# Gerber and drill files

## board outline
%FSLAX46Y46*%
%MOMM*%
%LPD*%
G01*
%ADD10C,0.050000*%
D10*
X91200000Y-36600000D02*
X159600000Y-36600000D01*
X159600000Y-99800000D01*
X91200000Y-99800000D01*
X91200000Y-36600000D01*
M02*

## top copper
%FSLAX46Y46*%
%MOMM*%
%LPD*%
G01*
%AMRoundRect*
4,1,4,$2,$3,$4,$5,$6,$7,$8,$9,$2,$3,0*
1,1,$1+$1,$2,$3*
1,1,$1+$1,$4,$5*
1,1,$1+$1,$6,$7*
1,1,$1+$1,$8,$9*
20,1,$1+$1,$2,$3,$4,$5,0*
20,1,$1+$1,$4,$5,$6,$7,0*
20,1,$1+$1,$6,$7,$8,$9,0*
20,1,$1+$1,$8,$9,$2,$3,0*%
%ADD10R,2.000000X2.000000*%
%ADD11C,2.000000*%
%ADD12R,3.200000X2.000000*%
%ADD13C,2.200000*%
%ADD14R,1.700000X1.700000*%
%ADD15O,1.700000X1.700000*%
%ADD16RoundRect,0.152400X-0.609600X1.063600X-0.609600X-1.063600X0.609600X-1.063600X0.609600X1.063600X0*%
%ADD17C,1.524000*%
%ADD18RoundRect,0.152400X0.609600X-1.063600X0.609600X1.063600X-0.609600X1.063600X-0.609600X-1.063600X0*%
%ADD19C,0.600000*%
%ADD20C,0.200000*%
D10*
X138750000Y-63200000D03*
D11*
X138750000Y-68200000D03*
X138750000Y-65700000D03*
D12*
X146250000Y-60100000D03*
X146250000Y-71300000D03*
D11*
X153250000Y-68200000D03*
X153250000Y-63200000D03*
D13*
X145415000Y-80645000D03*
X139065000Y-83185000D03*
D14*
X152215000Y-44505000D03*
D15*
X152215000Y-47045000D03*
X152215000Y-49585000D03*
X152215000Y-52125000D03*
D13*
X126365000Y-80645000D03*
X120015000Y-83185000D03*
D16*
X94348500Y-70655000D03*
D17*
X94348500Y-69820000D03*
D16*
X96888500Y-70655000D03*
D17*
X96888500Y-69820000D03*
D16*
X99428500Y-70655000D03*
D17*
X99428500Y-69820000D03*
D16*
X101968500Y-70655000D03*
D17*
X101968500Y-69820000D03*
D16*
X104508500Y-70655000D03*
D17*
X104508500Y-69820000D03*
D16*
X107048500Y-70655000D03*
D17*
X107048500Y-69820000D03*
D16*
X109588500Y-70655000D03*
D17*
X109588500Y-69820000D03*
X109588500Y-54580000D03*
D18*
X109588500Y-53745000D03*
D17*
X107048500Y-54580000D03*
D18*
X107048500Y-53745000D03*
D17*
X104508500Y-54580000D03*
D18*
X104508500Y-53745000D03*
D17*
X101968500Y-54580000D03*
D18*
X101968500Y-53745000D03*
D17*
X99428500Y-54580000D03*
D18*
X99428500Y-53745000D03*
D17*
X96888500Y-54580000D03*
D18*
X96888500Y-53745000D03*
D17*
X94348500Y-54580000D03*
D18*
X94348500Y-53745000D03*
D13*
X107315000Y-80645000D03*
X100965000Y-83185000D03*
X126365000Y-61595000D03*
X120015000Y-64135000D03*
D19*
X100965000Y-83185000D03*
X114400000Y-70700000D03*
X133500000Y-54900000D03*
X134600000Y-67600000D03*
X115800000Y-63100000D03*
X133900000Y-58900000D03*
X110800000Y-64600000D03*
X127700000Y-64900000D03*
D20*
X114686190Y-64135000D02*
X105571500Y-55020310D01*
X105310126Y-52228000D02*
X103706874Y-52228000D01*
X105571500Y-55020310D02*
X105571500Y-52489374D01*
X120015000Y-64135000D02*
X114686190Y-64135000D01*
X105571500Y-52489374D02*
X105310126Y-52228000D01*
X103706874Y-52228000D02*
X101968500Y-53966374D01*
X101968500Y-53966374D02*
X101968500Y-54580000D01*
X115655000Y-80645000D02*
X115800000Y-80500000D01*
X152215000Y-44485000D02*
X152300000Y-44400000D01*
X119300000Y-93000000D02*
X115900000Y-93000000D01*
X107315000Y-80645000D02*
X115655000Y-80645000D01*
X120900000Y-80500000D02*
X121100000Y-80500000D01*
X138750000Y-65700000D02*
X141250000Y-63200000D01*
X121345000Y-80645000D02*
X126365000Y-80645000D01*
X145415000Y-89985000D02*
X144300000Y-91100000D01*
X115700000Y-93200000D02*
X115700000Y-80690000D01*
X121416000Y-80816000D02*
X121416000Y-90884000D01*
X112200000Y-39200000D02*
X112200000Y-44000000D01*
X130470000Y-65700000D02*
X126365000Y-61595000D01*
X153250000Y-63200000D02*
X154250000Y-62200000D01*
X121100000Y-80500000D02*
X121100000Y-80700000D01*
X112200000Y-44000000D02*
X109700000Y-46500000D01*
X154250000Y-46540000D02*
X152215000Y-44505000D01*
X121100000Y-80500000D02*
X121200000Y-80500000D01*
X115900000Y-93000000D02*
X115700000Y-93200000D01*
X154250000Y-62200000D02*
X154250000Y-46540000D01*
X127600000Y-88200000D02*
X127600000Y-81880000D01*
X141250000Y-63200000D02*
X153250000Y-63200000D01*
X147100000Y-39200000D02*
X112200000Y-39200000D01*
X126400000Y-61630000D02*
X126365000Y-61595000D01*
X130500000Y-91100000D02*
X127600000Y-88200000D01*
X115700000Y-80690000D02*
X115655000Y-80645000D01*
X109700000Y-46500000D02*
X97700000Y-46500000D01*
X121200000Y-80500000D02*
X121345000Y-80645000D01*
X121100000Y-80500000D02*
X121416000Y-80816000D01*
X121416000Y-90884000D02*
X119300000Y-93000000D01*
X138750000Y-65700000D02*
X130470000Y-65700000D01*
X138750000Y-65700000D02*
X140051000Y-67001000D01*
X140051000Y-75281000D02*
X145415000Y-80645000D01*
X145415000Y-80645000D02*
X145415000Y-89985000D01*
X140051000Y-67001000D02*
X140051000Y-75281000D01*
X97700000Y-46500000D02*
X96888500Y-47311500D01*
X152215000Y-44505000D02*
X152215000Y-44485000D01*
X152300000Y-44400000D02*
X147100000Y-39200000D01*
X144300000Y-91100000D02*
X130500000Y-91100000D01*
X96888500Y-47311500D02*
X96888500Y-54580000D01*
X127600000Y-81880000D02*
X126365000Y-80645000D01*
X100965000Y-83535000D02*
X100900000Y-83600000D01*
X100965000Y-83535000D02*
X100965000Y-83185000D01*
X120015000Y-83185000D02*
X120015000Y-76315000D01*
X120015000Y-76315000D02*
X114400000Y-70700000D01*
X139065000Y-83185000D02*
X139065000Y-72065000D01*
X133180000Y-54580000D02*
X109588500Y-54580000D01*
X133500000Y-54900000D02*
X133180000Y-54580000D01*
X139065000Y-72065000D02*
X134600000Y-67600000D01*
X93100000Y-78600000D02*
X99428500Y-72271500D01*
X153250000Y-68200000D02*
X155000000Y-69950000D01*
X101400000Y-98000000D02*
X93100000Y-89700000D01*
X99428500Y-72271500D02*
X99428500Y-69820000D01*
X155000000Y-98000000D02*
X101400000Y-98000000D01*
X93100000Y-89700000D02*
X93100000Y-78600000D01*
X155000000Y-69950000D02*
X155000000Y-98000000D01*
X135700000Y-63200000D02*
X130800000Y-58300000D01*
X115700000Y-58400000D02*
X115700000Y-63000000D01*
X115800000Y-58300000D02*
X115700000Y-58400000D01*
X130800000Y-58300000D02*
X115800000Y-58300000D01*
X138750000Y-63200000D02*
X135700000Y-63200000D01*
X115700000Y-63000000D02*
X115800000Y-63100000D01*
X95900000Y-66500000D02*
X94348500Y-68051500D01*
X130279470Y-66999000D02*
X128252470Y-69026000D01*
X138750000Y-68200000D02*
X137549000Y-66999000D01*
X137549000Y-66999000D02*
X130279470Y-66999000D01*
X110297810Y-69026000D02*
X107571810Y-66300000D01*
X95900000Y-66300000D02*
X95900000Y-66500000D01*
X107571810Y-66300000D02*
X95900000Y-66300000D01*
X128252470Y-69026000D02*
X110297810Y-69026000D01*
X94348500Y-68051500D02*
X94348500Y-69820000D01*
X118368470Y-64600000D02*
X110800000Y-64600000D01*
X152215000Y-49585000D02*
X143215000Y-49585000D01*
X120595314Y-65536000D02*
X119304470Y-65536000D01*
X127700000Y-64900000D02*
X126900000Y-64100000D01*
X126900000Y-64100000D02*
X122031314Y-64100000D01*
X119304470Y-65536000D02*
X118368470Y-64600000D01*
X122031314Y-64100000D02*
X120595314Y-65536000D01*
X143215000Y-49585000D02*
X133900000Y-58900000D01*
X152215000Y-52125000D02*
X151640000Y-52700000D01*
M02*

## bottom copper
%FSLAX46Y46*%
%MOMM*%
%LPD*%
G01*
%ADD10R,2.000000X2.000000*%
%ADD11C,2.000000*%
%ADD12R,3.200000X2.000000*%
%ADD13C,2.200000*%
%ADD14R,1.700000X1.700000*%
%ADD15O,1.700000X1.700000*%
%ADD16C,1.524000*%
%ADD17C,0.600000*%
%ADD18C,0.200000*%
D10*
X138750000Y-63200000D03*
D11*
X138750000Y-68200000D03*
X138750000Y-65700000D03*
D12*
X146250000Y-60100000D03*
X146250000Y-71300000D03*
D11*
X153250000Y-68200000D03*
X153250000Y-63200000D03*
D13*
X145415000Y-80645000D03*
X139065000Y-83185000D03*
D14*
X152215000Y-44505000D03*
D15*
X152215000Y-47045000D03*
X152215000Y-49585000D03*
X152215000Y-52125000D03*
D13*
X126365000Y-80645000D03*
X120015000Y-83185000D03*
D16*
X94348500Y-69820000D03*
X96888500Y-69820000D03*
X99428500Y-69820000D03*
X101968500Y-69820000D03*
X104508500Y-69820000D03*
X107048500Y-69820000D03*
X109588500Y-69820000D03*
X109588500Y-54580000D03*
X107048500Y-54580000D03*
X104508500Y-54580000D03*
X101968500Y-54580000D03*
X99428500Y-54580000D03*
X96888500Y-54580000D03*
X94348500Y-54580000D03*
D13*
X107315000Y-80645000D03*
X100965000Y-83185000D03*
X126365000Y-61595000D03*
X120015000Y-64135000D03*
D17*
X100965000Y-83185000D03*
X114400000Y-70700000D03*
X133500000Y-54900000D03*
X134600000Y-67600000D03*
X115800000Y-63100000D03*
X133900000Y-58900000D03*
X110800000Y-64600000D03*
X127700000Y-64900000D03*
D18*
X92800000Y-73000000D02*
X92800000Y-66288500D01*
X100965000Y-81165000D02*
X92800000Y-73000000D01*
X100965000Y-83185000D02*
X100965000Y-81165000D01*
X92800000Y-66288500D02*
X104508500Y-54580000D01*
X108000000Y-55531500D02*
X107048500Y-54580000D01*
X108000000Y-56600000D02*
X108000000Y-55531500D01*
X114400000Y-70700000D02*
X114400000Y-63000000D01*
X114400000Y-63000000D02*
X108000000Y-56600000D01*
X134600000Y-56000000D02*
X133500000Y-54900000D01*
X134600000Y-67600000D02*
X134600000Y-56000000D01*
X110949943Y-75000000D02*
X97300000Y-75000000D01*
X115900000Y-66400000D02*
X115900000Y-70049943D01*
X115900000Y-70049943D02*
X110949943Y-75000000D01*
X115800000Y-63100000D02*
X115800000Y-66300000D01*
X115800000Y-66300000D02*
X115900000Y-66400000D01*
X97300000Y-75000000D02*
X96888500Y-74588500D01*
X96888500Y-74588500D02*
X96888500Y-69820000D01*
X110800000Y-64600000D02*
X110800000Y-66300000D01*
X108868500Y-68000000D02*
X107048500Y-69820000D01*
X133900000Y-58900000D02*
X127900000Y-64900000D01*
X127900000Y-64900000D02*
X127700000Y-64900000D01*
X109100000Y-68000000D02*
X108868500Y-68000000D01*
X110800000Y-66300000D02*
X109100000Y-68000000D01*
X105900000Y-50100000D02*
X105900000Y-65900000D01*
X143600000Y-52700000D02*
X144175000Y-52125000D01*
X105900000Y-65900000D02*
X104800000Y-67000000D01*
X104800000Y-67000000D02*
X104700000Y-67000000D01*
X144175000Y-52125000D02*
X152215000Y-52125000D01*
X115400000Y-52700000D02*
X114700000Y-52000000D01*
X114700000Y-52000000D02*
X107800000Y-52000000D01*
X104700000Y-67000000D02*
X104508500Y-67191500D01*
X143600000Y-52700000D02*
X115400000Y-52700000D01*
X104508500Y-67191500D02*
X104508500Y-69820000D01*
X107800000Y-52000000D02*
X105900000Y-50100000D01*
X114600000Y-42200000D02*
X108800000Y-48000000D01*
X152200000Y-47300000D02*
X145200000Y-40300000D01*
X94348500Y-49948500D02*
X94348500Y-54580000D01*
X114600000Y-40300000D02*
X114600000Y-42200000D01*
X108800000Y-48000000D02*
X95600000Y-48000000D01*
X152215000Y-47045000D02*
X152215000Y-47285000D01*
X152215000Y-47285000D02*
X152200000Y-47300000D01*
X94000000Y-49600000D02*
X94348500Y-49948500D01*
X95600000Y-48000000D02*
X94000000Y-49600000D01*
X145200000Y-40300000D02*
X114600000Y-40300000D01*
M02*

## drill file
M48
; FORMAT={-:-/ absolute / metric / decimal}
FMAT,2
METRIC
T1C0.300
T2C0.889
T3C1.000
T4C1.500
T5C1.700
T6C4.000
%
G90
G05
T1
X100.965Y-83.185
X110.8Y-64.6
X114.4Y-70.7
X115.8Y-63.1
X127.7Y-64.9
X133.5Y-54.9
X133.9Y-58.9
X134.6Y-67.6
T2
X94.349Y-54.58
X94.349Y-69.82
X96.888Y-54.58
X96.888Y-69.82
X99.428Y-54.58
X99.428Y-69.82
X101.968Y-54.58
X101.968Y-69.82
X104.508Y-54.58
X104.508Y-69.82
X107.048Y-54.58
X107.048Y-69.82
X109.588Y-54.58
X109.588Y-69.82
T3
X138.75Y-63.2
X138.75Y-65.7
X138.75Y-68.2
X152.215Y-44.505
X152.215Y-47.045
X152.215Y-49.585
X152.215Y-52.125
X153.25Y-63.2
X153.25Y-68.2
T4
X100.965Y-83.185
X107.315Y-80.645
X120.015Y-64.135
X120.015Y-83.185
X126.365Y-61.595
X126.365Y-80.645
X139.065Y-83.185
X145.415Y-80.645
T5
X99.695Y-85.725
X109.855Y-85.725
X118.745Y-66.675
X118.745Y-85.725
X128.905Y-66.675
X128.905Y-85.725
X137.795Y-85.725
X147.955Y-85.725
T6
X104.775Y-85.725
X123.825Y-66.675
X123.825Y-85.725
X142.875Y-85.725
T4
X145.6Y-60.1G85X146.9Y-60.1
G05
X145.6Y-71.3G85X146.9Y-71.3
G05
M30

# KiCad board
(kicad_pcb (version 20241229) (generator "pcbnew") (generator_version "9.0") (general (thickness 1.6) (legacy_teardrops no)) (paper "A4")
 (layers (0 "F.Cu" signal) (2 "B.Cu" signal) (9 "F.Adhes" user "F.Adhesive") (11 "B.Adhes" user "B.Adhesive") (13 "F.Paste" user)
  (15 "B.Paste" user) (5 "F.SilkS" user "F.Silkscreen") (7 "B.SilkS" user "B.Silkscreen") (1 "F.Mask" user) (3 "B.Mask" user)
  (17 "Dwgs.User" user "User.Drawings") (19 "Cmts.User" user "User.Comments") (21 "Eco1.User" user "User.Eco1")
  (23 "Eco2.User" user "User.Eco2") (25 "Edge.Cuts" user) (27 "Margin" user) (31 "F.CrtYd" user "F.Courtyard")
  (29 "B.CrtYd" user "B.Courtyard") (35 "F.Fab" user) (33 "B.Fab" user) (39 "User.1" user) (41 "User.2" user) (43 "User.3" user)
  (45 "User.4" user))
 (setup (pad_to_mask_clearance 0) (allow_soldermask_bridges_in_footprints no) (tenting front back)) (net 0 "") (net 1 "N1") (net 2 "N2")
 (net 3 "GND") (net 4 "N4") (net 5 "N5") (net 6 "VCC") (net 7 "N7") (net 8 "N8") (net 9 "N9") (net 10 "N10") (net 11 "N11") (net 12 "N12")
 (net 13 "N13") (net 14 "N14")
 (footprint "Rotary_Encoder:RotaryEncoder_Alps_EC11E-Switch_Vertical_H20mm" (layer "F.Cu") (at 138.75 63.2)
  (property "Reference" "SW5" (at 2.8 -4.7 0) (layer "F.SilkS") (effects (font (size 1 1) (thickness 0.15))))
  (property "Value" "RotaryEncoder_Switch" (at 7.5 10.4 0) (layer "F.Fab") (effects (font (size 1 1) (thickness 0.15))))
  (pad "A" thru_hole rect (at 0 0) (size 2 2) (drill 1) (layers "*.Cu" "*.Mask") (remove_unused_layers no) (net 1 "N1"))
  (pad "B" thru_hole circle (at 0 5) (size 2 2) (drill 1) (layers "*.Cu" "*.Mask") (remove_unused_layers no) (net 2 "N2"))
  (pad "C" thru_hole circle (at 0 2.5) (size 2 2) (drill 1) (layers "*.Cu" "*.Mask") (remove_unused_layers no) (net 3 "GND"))
  (pad "MP" thru_hole rect (at 7.5 -3.1) (size 3.2 2) (drill oval 2.8 1.5) (layers "*.Cu" "*.Mask") (remove_unused_layers no))
  (pad "MP" thru_hole rect (at 7.5 8.1) (size 3.2 2) (drill oval 2.8 1.5) (layers "*.Cu" "*.Mask") (remove_unused_layers no))
  (pad "S1" thru_hole circle (at 14.5 5) (size 2 2) (drill 1) (layers "*.Cu" "*.Mask") (remove_unused_layers no) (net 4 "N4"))
  (pad "S2" thru_hole circle (at 14.5 0) (size 2 2) (drill 1) (layers "*.Cu" "*.Mask") (remove_unused_layers no) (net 3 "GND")))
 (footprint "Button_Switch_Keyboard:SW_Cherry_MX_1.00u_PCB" (layer "F.Cu") (at 145.415 80.645)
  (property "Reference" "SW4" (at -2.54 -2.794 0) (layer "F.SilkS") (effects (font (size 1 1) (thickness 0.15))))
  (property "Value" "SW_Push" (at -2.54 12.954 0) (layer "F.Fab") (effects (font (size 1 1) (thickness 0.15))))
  (pad "" np_thru_hole circle (at -7.62 5.08) (size 1.7 1.7) (drill 1.7) (layers "*.Cu" "*.Mask"))
  (pad "" np_thru_hole circle (at -2.54 5.08) (size 4 4) (drill 4) (layers "*.Cu" "*.Mask"))
  (pad "" np_thru_hole circle (at 2.54 5.08) (size 1.7 1.7) (drill 1.7) (layers "*.Cu" "*.Mask"))
  (pad "1" thru_hole circle (at 0 0) (size 2.2 2.2) (drill 1.5) (layers "*.Cu" "*.Mask") (remove_unused_layers no) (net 3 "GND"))
  (pad "2" thru_hole circle (at -6.35 2.54) (size 2.2 2.2) (drill 1.5) (layers "*.Cu" "*.Mask") (remove_unused_layers no) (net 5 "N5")))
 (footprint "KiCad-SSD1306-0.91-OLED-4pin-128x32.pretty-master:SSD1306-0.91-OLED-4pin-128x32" (layer "F.Cu") (at 115.715 42.315)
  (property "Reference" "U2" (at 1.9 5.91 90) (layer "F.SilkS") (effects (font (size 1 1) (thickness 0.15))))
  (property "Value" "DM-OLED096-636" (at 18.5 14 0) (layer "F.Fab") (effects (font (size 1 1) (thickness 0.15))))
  (pad "1" thru_hole rect (at 36.5 2.19) (size 1.7 1.7) (drill 1) (layers "*.Cu" "*.Mask") (remove_unused_layers no) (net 3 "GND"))
  (pad "2" thru_hole oval (at 36.5 4.73) (size 1.7 1.7) (drill 1) (layers "*.Cu" "*.Mask") (remove_unused_layers no) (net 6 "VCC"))
  (pad "3" thru_hole oval (at 36.5 7.27) (size 1.7 1.7) (drill 1) (layers "*.Cu" "*.Mask") (remove_unused_layers no) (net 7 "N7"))
  (pad "4" thru_hole oval (at 36.5 9.81) (size 1.7 1.7) (drill 1) (layers "*.Cu" "*.Mask") (remove_unused_layers no) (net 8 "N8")))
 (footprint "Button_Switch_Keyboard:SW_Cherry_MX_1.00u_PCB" (layer "F.Cu") (at 126.365 80.645)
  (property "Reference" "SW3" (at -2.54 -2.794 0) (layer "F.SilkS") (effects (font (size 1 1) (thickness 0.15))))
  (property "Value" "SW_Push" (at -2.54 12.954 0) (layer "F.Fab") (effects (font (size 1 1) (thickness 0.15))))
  (pad "" np_thru_hole circle (at -7.62 5.08) (size 1.7 1.7) (drill 1.7) (layers "*.Cu" "*.Mask"))
  (pad "" np_thru_hole circle (at -2.54 5.08) (size 4 4) (drill 4) (layers "*.Cu" "*.Mask"))
  (pad "" np_thru_hole circle (at 2.54 5.08) (size 1.7 1.7) (drill 1.7) (layers "*.Cu" "*.Mask"))
  (pad "1" thru_hole circle (at 0 0) (size 2.2 2.2) (drill 1.5) (layers "*.Cu" "*.Mask") (remove_unused_layers no) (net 3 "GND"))
  (pad "2" thru_hole circle (at -6.35 2.54) (size 2.2 2.2) (drill 1.5) (layers "*.Cu" "*.Mask") (remove_unused_layers no) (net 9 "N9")))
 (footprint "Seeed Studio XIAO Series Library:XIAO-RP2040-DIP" (layer "F.Cu") (at 101.9685 62.2 90)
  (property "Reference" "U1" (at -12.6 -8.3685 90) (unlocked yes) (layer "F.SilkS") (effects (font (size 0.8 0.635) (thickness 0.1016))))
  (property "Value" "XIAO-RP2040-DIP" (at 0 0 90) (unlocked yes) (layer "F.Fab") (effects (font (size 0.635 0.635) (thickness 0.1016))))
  (pad "1" smd roundrect (at -8.455 -7.62 270) (size 2.432 1.524) (layers "F.Cu" "F.Mask") (roundrect_rratio 0.1) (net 2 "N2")
   (thermal_bridge_angle 45))
  (pad "1" thru_hole circle (at -7.62 -7.62 270) (size 1.524 1.524) (drill 0.889) (layers "*.Cu" "*.Mask") (remove_unused_layers no)
   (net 2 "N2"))
  (pad "2" smd roundrect (at -8.455 -5.08 270) (size 2.432 1.524) (layers "F.Cu" "F.Mask") (roundrect_rratio 0.1) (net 1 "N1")
   (thermal_bridge_angle 45))
  (pad "2" thru_hole circle (at -7.62 -5.08 270) (size 1.524 1.524) (drill 0.889) (layers "*.Cu" "*.Mask") (remove_unused_layers no)
   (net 1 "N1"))
  (pad "3" smd roundrect (at -8.455 -2.54 270) (size 2.432 1.524) (layers "F.Cu" "F.Mask") (roundrect_rratio 0.1) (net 4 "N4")
   (thermal_bridge_angle 45))
  (pad "3" thru_hole circle (at -7.62 -2.54 270) (size 1.524 1.524) (drill 0.889) (layers "*.Cu" "*.Mask") (remove_unused_layers no)
   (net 4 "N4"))
  (pad "4" smd roundrect (at -8.455 0 270) (size 2.432 1.524) (layers "F.Cu" "F.Mask") (roundrect_rratio 0.1) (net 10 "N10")
   (thermal_bridge_angle 45))
  (pad "4" thru_hole circle (at -7.62 0 270) (size 1.524 1.524) (drill 0.889) (layers "*.Cu" "*.Mask") (remove_unused_layers no)
   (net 10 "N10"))
  (pad "5" smd roundrect (at -8.455 2.54 270) (size 2.432 1.524) (layers "F.Cu" "F.Mask") (roundrect_rratio 0.1) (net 8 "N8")
   (thermal_bridge_angle 45))
  (pad "5" thru_hole circle (at -7.62 2.54 270) (size 1.524 1.524) (drill 0.889) (layers "*.Cu" "*.Mask") (remove_unused_layers no)
   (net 8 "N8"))
  (pad "6" smd roundrect (at -8.455 5.08 270) (size 2.432 1.524) (layers "F.Cu" "F.Mask") (roundrect_rratio 0.1) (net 7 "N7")
   (thermal_bridge_angle 45))
  (pad "6" thru_hole circle (at -7.62 5.08 270) (size 1.524 1.524) (drill 0.889) (layers "*.Cu" "*.Mask") (remove_unused_layers no)
   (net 7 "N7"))
  (pad "7" smd roundrect (at -8.455 7.62 270) (size 2.432 1.524) (layers "F.Cu" "F.Mask") (roundrect_rratio 0.1) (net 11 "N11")
   (thermal_bridge_angle 45))
  (pad "7" thru_hole circle (at -7.62 7.62 270) (size 1.524 1.524) (drill 0.889) (layers "*.Cu" "*.Mask") (remove_unused_layers no)
   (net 11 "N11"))
  (pad "8" thru_hole circle (at 7.62 7.62 90) (size 1.524 1.524) (drill 0.889) (layers "*.Cu" "*.Mask") (remove_unused_layers no)
   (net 5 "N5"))
  (pad "8" smd roundrect (at 8.455 7.62 90) (size 2.432 1.524) (layers "F.Cu" "F.Mask") (roundrect_rratio 0.1) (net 5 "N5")
   (thermal_bridge_angle 45))
  (pad "9" thru_hole circle (at 7.62 5.08 90) (size 1.524 1.524) (drill 0.889) (layers "*.Cu" "*.Mask") (remove_unused_layers no)
   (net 9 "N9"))
  (pad "9" smd roundrect (at 8.455 5.08 90) (size 2.432 1.524) (layers "F.Cu" "F.Mask") (roundrect_rratio 0.1) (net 9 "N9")
   (thermal_bridge_angle 45))
  (pad "10" thru_hole circle (at 7.62 2.54 90) (size 1.524 1.524) (drill 0.889) (layers "*.Cu" "*.Mask") (remove_unused_layers no)
   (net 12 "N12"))
  (pad "10" smd roundrect (at 8.455 2.54 90) (size 2.432 1.524) (layers "F.Cu" "F.Mask") (roundrect_rratio 0.1) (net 12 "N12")
   (thermal_bridge_angle 45))
  (pad "11" thru_hole circle (at 7.62 0 90) (size 1.524 1.524) (drill 0.889) (layers "*.Cu" "*.Mask") (remove_unused_layers no)
   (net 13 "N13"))
  (pad "11" smd roundrect (at 8.455 0 90) (size 2.432 1.524) (layers "F.Cu" "F.Mask") (roundrect_rratio 0.1) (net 13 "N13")
   (thermal_bridge_angle 45))
  (pad "12" thru_hole circle (at 7.62 -2.54 90) (size 1.524 1.524) (drill 0.889) (layers "*.Cu" "*.Mask") (remove_unused_layers no)
   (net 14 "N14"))
  (pad "12" smd roundrect (at 8.455 -2.54 90) (size 2.432 1.524) (layers "F.Cu" "F.Mask") (roundrect_rratio 0.1) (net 14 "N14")
   (thermal_bridge_angle 45))
  (pad "13" thru_hole circle (at 7.62 -5.08 90) (size 1.524 1.524) (drill 0.889) (layers "*.Cu" "*.Mask") (remove_unused_layers no)
   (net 3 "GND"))
  (pad "13" smd roundrect (at 8.455 -5.08 90) (size 2.432 1.524) (layers "F.Cu" "F.Mask") (roundrect_rratio 0.1) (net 3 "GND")
   (thermal_bridge_angle 45))
  (pad "14" thru_hole circle (at 7.62 -7.62 90) (size 1.524 1.524) (drill 0.889) (layers "*.Cu" "*.Mask") (remove_unused_layers no)
   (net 6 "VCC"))
  (pad "14" smd roundrect (at 8.455 -7.62 90) (size 2.432 1.524) (layers "F.Cu" "F.Mask") (roundrect_rratio 0.1) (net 6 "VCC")
   (thermal_bridge_angle 45)))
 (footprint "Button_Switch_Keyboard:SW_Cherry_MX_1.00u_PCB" (layer "F.Cu") (at 107.315 80.645)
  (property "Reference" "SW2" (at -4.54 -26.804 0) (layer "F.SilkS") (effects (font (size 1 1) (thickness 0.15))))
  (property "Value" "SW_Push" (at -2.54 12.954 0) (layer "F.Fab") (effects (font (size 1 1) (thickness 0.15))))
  (pad "" np_thru_hole circle (at -7.62 5.08) (size 1.7 1.7) (drill 1.7) (layers "*.Cu" "*.Mask"))
  (pad "" np_thru_hole circle (at -2.54 5.08) (size 4 4) (drill 4) (layers "*.Cu" "*.Mask"))
  (pad "" np_thru_hole circle (at 2.54 5.08) (size 1.7 1.7) (drill 1.7) (layers "*.Cu" "*.Mask"))
  (pad "1" thru_hole circle (at 0 0) (size 2.2 2.2) (drill 1.5) (layers "*.Cu" "*.Mask") (remove_unused_layers no) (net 3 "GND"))
  (pad "2" thru_hole circle (at -6.35 2.54) (size 2.2 2.2) (drill 1.5) (layers "*.Cu" "*.Mask") (remove_unused_layers no) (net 12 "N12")))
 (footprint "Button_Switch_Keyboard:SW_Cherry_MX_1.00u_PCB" (layer "F.Cu") (at 126.365 61.595)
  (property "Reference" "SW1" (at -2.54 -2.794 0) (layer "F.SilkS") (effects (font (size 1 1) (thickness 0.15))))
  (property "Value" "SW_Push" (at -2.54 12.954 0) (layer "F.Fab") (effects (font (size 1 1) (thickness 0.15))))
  (pad "" np_thru_hole circle (at -7.62 5.08) (size 1.7 1.7) (drill 1.7) (layers "*.Cu" "*.Mask"))
  (pad "" np_thru_hole circle (at -2.54 5.08) (size 4 4) (drill 4) (layers "*.Cu" "*.Mask"))
  (pad "" np_thru_hole circle (at 2.54 5.08) (size 1.7 1.7) (drill 1.7) (layers "*.Cu" "*.Mask"))
  (pad "1" thru_hole circle (at 0 0) (size 2.2 2.2) (drill 1.5) (layers "*.Cu" "*.Mask") (remove_unused_layers no) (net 3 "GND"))
  (pad "2" thru_hole circle (at -6.35 2.54) (size 2.2 2.2) (drill 1.5) (layers "*.Cu" "*.Mask") (remove_unused_layers no) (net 13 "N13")))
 (gr_rect (start 91.2 36.6) (end 159.6 99.8) (stroke (width 0.05) (type default)) (fill no) (layer "Edge.Cuts"))
 (segment (start 114.68619 64.135) (end 105.5715 55.02031) (width 0.2) (layer "F.Cu") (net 13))
 (segment (start 105.310126 52.228) (end 103.706874 52.228) (width 0.2) (layer "F.Cu") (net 13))
 (segment (start 105.5715 55.02031) (end 105.5715 52.489374) (width 0.2) (layer "F.Cu") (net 13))
 (segment (start 120.015 64.135) (end 114.68619 64.135) (width 0.2) (layer "F.Cu") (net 13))
 (segment (start 105.5715 52.489374) (end 105.310126 52.228) (width 0.2) (layer "F.Cu") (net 13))
 (segment (start 103.706874 52.228) (end 101.9685 53.966374) (width 0.2) (layer "F.Cu") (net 13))
 (segment (start 101.9685 53.966374) (end 101.9685 54.58) (width 0.2) (layer "F.Cu") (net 13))
 (segment (start 115.655 80.645) (end 115.8 80.5) (width 0.2) (layer "F.Cu") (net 3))
 (segment (start 152.215 44.485) (end 152.3 44.4) (width 0.2) (layer "F.Cu") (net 3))
 (segment (start 119.3 93) (end 115.9 93) (width 0.2) (layer "F.Cu") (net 3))
 (segment (start 107.315 80.645) (end 115.655 80.645) (width 0.2) (layer "F.Cu") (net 3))
 (segment (start 120.9 80.5) (end 121.1 80.5) (width 0.2) (layer "F.Cu") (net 3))
 (segment (start 138.75 65.7) (end 141.25 63.2) (width 0.2) (layer "F.Cu") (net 3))
 (segment (start 121.345 80.645) (end 126.365 80.645) (width 0.2) (layer "F.Cu") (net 3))
 (segment (start 145.415 89.985) (end 144.3 91.1) (width 0.2) (layer "F.Cu") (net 3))
 (segment (start 115.7 93.2) (end 115.7 80.69) (width 0.2) (layer "F.Cu") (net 3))
 (segment (start 121.416 80.816) (end 121.416 90.884) (width 0.2) (layer "F.Cu") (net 3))
 (segment (start 112.2 39.2) (end 112.2 44) (width 0.2) (layer "F.Cu") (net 3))
 (segment (start 130.47 65.7) (end 126.365 61.595) (width 0.2) (layer "F.Cu") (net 3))
 (segment (start 153.25 63.2) (end 154.25 62.2) (width 0.2) (layer "F.Cu") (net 3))
 (segment (start 121.1 80.5) (end 121.1 80.7) (width 0.2) (layer "F.Cu") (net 3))
 (segment (start 112.2 44) (end 109.7 46.5) (width 0.2) (layer "F.Cu") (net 3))
 (segment (start 154.25 46.54) (end 152.215 44.505) (width 0.2) (layer "F.Cu") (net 3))
 (segment (start 121.1 80.5) (end 121.2 80.5) (width 0.2) (layer "F.Cu") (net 3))
 (segment (start 115.9 93) (end 115.7 93.2) (width 0.2) (layer "F.Cu") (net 3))
 (segment (start 154.25 62.2) (end 154.25 46.54) (width 0.2) (layer "F.Cu") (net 3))
 (segment (start 127.6 88.2) (end 127.6 81.88) (width 0.2) (layer "F.Cu") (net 3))
 (segment (start 141.25 63.2) (end 153.25 63.2) (width 0.2) (layer "F.Cu") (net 3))
 (segment (start 147.1 39.2) (end 112.2 39.2) (width 0.2) (layer "F.Cu") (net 3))
 (segment (start 126.4 61.63) (end 126.365 61.595) (width 0.2) (layer "F.Cu") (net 3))
 (segment (start 130.5 91.1) (end 127.6 88.2) (width 0.2) (layer "F.Cu") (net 3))
 (segment (start 115.7 80.69) (end 115.655 80.645) (width 0.2) (layer "F.Cu") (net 3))
 (segment (start 109.7 46.5) (end 97.7 46.5) (width 0.2) (layer "F.Cu") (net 3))
 (segment (start 121.2 80.5) (end 121.345 80.645) (width 0.2) (layer "F.Cu") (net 3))
 (segment (start 121.1 80.5) (end 121.416 80.816) (width 0.2) (layer "F.Cu") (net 3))
 (segment (start 121.416 90.884) (end 119.3 93) (width 0.2) (layer "F.Cu") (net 3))
 (segment (start 138.75 65.7) (end 130.47 65.7) (width 0.2) (layer "F.Cu") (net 3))
 (segment (start 138.75 65.7) (end 140.051 67.001) (width 0.2) (layer "F.Cu") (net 3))
 (segment (start 140.051 75.281) (end 145.415 80.645) (width 0.2) (layer "F.Cu") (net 3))
 (segment (start 145.415 80.645) (end 145.415 89.985) (width 0.2) (layer "F.Cu") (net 3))
 (segment (start 140.051 67.001) (end 140.051 75.281) (width 0.2) (layer "F.Cu") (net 3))
 (segment (start 97.7 46.5) (end 96.8885 47.3115) (width 0.2) (layer "F.Cu") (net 3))
 (segment (start 152.215 44.505) (end 152.215 44.485) (width 0.2) (layer "F.Cu") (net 3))
 (segment (start 152.3 44.4) (end 147.1 39.2) (width 0.2) (layer "F.Cu") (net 3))
 (segment (start 144.3 91.1) (end 130.5 91.1) (width 0.2) (layer "F.Cu") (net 3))
 (segment (start 96.8885 47.3115) (end 96.8885 54.58) (width 0.2) (layer "F.Cu") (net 3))
 (segment (start 127.6 81.88) (end 126.365 80.645) (width 0.2) (layer "F.Cu") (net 3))
 (segment (start 100.965 83.535) (end 100.9 83.6) (width 0.2) (layer "F.Cu") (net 12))
 (segment (start 100.965 83.535) (end 100.965 83.185) (width 0.2) (layer "F.Cu") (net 12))
 (via (at 100.965 83.185) (size 0.6) (drill 0.3) (layers "F.Cu" "B.Cu") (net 12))
 (segment (start 92.8 73) (end 92.8 66.2885) (width 0.2) (layer "B.Cu") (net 12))
 (segment (start 100.965 81.165) (end 92.8 73) (width 0.2) (layer "B.Cu") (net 12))
 (segment (start 100.965 83.185) (end 100.965 81.165) (width 0.2) (layer "B.Cu") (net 12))
 (segment (start 92.8 66.2885) (end 104.5085 54.58) (width 0.2) (layer "B.Cu") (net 12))
 (segment (start 120.015 83.185) (end 120.015 76.315) (width 0.2) (layer "F.Cu") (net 9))
 (segment (start 120.015 76.315) (end 114.4 70.7) (width 0.2) (layer "F.Cu") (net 9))
 (via (at 114.4 70.7) (size 0.6) (drill 0.3) (layers "F.Cu" "B.Cu") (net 9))
 (segment (start 108 55.5315) (end 107.0485 54.58) (width 0.2) (layer "B.Cu") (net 9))
 (segment (start 108 56.6) (end 108 55.5315) (width 0.2) (layer "B.Cu") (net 9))
 (segment (start 114.4 70.7) (end 114.4 63) (width 0.2) (layer "B.Cu") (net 9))
 (segment (start 114.4 63) (end 108 56.6) (width 0.2) (layer "B.Cu") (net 9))
 (segment (start 139.065 83.185) (end 139.065 72.065) (width 0.2) (layer "F.Cu") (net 5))
 (segment (start 133.18 54.58) (end 109.5885 54.58) (width 0.2) (layer "F.Cu") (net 5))
 (segment (start 133.5 54.9) (end 133.18 54.58) (width 0.2) (layer "F.Cu") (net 5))
 (segment (start 139.065 72.065) (end 134.6 67.6) (width 0.2) (layer "F.Cu") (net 5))
 (via (at 133.5 54.9) (size 0.6) (drill 0.3) (layers "F.Cu" "B.Cu") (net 5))
 (via (at 134.6 67.6) (size 0.6) (drill 0.3) (layers "F.Cu" "B.Cu") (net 5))
 (segment (start 134.6 56) (end 133.5 54.9) (width 0.2) (layer "B.Cu") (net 5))
 (segment (start 134.6 67.6) (end 134.6 56) (width 0.2) (layer "B.Cu") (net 5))
 (segment (start 93.1 78.6) (end 99.4285 72.2715) (width 0.2) (layer "F.Cu") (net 4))
 (segment (start 153.25 68.2) (end 155 69.95) (width 0.2) (layer "F.Cu") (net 4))
 (segment (start 101.4 98) (end 93.1 89.7) (width 0.2) (layer "F.Cu") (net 4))
 (segment (start 99.4285 72.2715) (end 99.4285 69.82) (width 0.2) (layer "F.Cu") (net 4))
 (segment (start 155 98) (end 101.4 98) (width 0.2) (layer "F.Cu") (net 4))
 (segment (start 93.1 89.7) (end 93.1 78.6) (width 0.2) (layer "F.Cu") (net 4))
 (segment (start 155 69.95) (end 155 98) (width 0.2) (layer "F.Cu") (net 4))
 (segment (start 135.7 63.2) (end 130.8 58.3) (width 0.2) (layer "F.Cu") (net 1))
 (segment (start 115.7 58.4) (end 115.7 63) (width 0.2) (layer "F.Cu") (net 1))
 (segment (start 115.8 58.3) (end 115.7 58.4) (width 0.2) (layer "F.Cu") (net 1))
 (segment (start 130.8 58.3) (end 115.8 58.3) (width 0.2) (layer "F.Cu") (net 1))
 (segment (start 138.75 63.2) (end 135.7 63.2) (width 0.2) (layer "F.Cu") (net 1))
 (segment (start 115.7 63) (end 115.8 63.1) (width 0.2) (layer "F.Cu") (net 1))
 (via (at 115.8 63.1) (size 0.6) (drill 0.3) (layers "F.Cu" "B.Cu") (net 1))
 (segment (start 110.949943 75) (end 97.3 75) (width 0.2) (layer "B.Cu") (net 1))
 (segment (start 115.9 66.4) (end 115.9 70.049943) (width 0.2) (layer "B.Cu") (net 1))
 (segment (start 115.9 70.049943) (end 110.949943 75) (width 0.2) (layer "B.Cu") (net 1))
 (segment (start 115.8 63.1) (end 115.8 66.3) (width 0.2) (layer "B.Cu") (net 1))
 (segment (start 115.8 66.3) (end 115.9 66.4) (width 0.2) (layer "B.Cu") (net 1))
 (segment (start 97.3 75) (end 96.8885 74.5885) (width 0.2) (layer "B.Cu") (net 1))
 (segment (start 96.8885 74.5885) (end 96.8885 69.82) (width 0.2) (layer "B.Cu") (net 1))
 (segment (start 95.9 66.5) (end 94.3485 68.0515) (width 0.2) (layer "F.Cu") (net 2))
 (segment (start 130.27947 66.999) (end 128.25247 69.026) (width 0.2) (layer "F.Cu") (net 2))
 (segment (start 138.75 68.2) (end 137.549 66.999) (width 0.2) (layer "F.Cu") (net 2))
 (segment (start 137.549 66.999) (end 130.27947 66.999) (width 0.2) (layer "F.Cu") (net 2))
 (segment (start 110.29781 69.026) (end 107.57181 66.3) (width 0.2) (layer "F.Cu") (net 2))
 (segment (start 95.9 66.3) (end 95.9 66.5) (width 0.2) (layer "F.Cu") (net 2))
 (segment (start 107.57181 66.3) (end 95.9 66.3) (width 0.2) (layer "F.Cu") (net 2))
 (segment (start 128.25247 69.026) (end 110.29781 69.026) (width 0.2) (layer "F.Cu") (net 2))
 (segment (start 94.3485 68.0515) (end 94.3485 69.82) (width 0.2) (layer "F.Cu") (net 2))
 (segment (start 118.36847 64.6) (end 110.8 64.6) (width 0.2) (layer "F.Cu") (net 7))
 (segment (start 152.215 49.585) (end 143.215 49.585) (width 0.2) (layer "F.Cu") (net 7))
 (segment (start 120.595314 65.536) (end 119.30447 65.536) (width 0.2) (layer "F.Cu") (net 7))
 (segment (start 127.7 64.9) (end 126.9 64.1) (width 0.2) (layer "F.Cu") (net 7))
 (segment (start 126.9 64.1) (end 122.031314 64.1) (width 0.2) (layer "F.Cu") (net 7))
 (segment (start 119.30447 65.536) (end 118.36847 64.6) (width 0.2) (layer "F.Cu") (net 7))
 (segment (start 122.031314 64.1) (end 120.595314 65.536) (width 0.2) (layer "F.Cu") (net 7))
 (segment (start 143.215 49.585) (end 133.9 58.9) (width 0.2) (layer "F.Cu") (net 7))
 (via (at 133.9 58.9) (size 0.6) (drill 0.3) (layers "F.Cu" "B.Cu") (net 7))
 (via (at 110.8 64.6) (size 0.6) (drill 0.3) (layers "F.Cu" "B.Cu") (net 7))
 (via (at 127.7 64.9) (size 0.6) (drill 0.3) (layers "F.Cu" "B.Cu") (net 7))
 (segment (start 110.8 64.6) (end 110.8 66.3) (width 0.2) (layer "B.Cu") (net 7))
 (segment (start 108.8685 68) (end 107.0485 69.82) (width 0.2) (layer "B.Cu") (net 7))
 (segment (start 133.9 58.9) (end 127.9 64.9) (width 0.2) (layer "B.Cu") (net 7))
 (segment (start 127.9 64.9) (end 127.7 64.9) (width 0.2) (layer "B.Cu") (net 7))
 (segment (start 109.1 68) (end 108.8685 68) (width 0.2) (layer "B.Cu") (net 7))
 (segment (start 110.8 66.3) (end 109.1 68) (width 0.2) (layer "B.Cu") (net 7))
 (segment (start 152.215 52.125) (end 151.64 52.7) (width 0.2) (layer "F.Cu") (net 8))
 (segment (start 105.9 50.1) (end 105.9 65.9) (width 0.2) (layer "B.Cu") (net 8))
 (segment (start 143.6 52.7) (end 144.175 52.125) (width 0.2) (layer "B.Cu") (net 8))
 (segment (start 105.9 65.9) (end 104.8 67) (width 0.2) (layer "B.Cu") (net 8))
 (segment (start 104.8 67) (end 104.7 67) (width 0.2) (layer "B.Cu") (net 8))
 (segment (start 144.175 52.125) (end 152.215 52.125) (width 0.2) (layer "B.Cu") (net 8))
 (segment (start 115.4 52.7) (end 114.7 52) (width 0.2) (layer "B.Cu") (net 8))
 (segment (start 114.7 52) (end 107.8 52) (width 0.2) (layer "B.Cu") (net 8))
 (segment (start 104.7 67) (end 104.5085 67.1915) (width 0.2) (layer "B.Cu") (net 8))
 (segment (start 143.6 52.7) (end 115.4 52.7) (width 0.2) (layer "B.Cu") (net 8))
 (segment (start 104.5085 67.1915) (end 104.5085 69.82) (width 0.2) (layer "B.Cu") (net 8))
 (segment (start 107.8 52) (end 105.9 50.1) (width 0.2) (layer "B.Cu") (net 8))
 (segment (start 114.6 42.2) (end 108.8 48) (width 0.2) (layer "B.Cu") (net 6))
 (segment (start 152.2 47.3) (end 145.2 40.3) (width 0.2) (layer "B.Cu") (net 6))
 (segment (start 94.3485 49.9485) (end 94.3485 54.58) (width 0.2) (layer "B.Cu") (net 6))
 (segment (start 114.6 40.3) (end 114.6 42.2) (width 0.2) (layer "B.Cu") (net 6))
 (segment (start 108.8 48) (end 95.6 48) (width 0.2) (layer "B.Cu") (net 6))
 (segment (start 152.215 47.045) (end 152.215 47.285) (width 0.2) (layer "B.Cu") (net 6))
 (segment (start 152.215 47.285) (end 152.2 47.3) (width 0.2) (layer "B.Cu") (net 6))
 (segment (start 94 49.6) (end 94.3485 49.9485) (width 0.2) (layer "B.Cu") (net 6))
 (segment (start 95.6 48) (end 94 49.6) (width 0.2) (layer "B.Cu") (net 6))
 (segment (start 145.2 40.3) (end 114.6 40.3) (width 0.2) (layer "B.Cu") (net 6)))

